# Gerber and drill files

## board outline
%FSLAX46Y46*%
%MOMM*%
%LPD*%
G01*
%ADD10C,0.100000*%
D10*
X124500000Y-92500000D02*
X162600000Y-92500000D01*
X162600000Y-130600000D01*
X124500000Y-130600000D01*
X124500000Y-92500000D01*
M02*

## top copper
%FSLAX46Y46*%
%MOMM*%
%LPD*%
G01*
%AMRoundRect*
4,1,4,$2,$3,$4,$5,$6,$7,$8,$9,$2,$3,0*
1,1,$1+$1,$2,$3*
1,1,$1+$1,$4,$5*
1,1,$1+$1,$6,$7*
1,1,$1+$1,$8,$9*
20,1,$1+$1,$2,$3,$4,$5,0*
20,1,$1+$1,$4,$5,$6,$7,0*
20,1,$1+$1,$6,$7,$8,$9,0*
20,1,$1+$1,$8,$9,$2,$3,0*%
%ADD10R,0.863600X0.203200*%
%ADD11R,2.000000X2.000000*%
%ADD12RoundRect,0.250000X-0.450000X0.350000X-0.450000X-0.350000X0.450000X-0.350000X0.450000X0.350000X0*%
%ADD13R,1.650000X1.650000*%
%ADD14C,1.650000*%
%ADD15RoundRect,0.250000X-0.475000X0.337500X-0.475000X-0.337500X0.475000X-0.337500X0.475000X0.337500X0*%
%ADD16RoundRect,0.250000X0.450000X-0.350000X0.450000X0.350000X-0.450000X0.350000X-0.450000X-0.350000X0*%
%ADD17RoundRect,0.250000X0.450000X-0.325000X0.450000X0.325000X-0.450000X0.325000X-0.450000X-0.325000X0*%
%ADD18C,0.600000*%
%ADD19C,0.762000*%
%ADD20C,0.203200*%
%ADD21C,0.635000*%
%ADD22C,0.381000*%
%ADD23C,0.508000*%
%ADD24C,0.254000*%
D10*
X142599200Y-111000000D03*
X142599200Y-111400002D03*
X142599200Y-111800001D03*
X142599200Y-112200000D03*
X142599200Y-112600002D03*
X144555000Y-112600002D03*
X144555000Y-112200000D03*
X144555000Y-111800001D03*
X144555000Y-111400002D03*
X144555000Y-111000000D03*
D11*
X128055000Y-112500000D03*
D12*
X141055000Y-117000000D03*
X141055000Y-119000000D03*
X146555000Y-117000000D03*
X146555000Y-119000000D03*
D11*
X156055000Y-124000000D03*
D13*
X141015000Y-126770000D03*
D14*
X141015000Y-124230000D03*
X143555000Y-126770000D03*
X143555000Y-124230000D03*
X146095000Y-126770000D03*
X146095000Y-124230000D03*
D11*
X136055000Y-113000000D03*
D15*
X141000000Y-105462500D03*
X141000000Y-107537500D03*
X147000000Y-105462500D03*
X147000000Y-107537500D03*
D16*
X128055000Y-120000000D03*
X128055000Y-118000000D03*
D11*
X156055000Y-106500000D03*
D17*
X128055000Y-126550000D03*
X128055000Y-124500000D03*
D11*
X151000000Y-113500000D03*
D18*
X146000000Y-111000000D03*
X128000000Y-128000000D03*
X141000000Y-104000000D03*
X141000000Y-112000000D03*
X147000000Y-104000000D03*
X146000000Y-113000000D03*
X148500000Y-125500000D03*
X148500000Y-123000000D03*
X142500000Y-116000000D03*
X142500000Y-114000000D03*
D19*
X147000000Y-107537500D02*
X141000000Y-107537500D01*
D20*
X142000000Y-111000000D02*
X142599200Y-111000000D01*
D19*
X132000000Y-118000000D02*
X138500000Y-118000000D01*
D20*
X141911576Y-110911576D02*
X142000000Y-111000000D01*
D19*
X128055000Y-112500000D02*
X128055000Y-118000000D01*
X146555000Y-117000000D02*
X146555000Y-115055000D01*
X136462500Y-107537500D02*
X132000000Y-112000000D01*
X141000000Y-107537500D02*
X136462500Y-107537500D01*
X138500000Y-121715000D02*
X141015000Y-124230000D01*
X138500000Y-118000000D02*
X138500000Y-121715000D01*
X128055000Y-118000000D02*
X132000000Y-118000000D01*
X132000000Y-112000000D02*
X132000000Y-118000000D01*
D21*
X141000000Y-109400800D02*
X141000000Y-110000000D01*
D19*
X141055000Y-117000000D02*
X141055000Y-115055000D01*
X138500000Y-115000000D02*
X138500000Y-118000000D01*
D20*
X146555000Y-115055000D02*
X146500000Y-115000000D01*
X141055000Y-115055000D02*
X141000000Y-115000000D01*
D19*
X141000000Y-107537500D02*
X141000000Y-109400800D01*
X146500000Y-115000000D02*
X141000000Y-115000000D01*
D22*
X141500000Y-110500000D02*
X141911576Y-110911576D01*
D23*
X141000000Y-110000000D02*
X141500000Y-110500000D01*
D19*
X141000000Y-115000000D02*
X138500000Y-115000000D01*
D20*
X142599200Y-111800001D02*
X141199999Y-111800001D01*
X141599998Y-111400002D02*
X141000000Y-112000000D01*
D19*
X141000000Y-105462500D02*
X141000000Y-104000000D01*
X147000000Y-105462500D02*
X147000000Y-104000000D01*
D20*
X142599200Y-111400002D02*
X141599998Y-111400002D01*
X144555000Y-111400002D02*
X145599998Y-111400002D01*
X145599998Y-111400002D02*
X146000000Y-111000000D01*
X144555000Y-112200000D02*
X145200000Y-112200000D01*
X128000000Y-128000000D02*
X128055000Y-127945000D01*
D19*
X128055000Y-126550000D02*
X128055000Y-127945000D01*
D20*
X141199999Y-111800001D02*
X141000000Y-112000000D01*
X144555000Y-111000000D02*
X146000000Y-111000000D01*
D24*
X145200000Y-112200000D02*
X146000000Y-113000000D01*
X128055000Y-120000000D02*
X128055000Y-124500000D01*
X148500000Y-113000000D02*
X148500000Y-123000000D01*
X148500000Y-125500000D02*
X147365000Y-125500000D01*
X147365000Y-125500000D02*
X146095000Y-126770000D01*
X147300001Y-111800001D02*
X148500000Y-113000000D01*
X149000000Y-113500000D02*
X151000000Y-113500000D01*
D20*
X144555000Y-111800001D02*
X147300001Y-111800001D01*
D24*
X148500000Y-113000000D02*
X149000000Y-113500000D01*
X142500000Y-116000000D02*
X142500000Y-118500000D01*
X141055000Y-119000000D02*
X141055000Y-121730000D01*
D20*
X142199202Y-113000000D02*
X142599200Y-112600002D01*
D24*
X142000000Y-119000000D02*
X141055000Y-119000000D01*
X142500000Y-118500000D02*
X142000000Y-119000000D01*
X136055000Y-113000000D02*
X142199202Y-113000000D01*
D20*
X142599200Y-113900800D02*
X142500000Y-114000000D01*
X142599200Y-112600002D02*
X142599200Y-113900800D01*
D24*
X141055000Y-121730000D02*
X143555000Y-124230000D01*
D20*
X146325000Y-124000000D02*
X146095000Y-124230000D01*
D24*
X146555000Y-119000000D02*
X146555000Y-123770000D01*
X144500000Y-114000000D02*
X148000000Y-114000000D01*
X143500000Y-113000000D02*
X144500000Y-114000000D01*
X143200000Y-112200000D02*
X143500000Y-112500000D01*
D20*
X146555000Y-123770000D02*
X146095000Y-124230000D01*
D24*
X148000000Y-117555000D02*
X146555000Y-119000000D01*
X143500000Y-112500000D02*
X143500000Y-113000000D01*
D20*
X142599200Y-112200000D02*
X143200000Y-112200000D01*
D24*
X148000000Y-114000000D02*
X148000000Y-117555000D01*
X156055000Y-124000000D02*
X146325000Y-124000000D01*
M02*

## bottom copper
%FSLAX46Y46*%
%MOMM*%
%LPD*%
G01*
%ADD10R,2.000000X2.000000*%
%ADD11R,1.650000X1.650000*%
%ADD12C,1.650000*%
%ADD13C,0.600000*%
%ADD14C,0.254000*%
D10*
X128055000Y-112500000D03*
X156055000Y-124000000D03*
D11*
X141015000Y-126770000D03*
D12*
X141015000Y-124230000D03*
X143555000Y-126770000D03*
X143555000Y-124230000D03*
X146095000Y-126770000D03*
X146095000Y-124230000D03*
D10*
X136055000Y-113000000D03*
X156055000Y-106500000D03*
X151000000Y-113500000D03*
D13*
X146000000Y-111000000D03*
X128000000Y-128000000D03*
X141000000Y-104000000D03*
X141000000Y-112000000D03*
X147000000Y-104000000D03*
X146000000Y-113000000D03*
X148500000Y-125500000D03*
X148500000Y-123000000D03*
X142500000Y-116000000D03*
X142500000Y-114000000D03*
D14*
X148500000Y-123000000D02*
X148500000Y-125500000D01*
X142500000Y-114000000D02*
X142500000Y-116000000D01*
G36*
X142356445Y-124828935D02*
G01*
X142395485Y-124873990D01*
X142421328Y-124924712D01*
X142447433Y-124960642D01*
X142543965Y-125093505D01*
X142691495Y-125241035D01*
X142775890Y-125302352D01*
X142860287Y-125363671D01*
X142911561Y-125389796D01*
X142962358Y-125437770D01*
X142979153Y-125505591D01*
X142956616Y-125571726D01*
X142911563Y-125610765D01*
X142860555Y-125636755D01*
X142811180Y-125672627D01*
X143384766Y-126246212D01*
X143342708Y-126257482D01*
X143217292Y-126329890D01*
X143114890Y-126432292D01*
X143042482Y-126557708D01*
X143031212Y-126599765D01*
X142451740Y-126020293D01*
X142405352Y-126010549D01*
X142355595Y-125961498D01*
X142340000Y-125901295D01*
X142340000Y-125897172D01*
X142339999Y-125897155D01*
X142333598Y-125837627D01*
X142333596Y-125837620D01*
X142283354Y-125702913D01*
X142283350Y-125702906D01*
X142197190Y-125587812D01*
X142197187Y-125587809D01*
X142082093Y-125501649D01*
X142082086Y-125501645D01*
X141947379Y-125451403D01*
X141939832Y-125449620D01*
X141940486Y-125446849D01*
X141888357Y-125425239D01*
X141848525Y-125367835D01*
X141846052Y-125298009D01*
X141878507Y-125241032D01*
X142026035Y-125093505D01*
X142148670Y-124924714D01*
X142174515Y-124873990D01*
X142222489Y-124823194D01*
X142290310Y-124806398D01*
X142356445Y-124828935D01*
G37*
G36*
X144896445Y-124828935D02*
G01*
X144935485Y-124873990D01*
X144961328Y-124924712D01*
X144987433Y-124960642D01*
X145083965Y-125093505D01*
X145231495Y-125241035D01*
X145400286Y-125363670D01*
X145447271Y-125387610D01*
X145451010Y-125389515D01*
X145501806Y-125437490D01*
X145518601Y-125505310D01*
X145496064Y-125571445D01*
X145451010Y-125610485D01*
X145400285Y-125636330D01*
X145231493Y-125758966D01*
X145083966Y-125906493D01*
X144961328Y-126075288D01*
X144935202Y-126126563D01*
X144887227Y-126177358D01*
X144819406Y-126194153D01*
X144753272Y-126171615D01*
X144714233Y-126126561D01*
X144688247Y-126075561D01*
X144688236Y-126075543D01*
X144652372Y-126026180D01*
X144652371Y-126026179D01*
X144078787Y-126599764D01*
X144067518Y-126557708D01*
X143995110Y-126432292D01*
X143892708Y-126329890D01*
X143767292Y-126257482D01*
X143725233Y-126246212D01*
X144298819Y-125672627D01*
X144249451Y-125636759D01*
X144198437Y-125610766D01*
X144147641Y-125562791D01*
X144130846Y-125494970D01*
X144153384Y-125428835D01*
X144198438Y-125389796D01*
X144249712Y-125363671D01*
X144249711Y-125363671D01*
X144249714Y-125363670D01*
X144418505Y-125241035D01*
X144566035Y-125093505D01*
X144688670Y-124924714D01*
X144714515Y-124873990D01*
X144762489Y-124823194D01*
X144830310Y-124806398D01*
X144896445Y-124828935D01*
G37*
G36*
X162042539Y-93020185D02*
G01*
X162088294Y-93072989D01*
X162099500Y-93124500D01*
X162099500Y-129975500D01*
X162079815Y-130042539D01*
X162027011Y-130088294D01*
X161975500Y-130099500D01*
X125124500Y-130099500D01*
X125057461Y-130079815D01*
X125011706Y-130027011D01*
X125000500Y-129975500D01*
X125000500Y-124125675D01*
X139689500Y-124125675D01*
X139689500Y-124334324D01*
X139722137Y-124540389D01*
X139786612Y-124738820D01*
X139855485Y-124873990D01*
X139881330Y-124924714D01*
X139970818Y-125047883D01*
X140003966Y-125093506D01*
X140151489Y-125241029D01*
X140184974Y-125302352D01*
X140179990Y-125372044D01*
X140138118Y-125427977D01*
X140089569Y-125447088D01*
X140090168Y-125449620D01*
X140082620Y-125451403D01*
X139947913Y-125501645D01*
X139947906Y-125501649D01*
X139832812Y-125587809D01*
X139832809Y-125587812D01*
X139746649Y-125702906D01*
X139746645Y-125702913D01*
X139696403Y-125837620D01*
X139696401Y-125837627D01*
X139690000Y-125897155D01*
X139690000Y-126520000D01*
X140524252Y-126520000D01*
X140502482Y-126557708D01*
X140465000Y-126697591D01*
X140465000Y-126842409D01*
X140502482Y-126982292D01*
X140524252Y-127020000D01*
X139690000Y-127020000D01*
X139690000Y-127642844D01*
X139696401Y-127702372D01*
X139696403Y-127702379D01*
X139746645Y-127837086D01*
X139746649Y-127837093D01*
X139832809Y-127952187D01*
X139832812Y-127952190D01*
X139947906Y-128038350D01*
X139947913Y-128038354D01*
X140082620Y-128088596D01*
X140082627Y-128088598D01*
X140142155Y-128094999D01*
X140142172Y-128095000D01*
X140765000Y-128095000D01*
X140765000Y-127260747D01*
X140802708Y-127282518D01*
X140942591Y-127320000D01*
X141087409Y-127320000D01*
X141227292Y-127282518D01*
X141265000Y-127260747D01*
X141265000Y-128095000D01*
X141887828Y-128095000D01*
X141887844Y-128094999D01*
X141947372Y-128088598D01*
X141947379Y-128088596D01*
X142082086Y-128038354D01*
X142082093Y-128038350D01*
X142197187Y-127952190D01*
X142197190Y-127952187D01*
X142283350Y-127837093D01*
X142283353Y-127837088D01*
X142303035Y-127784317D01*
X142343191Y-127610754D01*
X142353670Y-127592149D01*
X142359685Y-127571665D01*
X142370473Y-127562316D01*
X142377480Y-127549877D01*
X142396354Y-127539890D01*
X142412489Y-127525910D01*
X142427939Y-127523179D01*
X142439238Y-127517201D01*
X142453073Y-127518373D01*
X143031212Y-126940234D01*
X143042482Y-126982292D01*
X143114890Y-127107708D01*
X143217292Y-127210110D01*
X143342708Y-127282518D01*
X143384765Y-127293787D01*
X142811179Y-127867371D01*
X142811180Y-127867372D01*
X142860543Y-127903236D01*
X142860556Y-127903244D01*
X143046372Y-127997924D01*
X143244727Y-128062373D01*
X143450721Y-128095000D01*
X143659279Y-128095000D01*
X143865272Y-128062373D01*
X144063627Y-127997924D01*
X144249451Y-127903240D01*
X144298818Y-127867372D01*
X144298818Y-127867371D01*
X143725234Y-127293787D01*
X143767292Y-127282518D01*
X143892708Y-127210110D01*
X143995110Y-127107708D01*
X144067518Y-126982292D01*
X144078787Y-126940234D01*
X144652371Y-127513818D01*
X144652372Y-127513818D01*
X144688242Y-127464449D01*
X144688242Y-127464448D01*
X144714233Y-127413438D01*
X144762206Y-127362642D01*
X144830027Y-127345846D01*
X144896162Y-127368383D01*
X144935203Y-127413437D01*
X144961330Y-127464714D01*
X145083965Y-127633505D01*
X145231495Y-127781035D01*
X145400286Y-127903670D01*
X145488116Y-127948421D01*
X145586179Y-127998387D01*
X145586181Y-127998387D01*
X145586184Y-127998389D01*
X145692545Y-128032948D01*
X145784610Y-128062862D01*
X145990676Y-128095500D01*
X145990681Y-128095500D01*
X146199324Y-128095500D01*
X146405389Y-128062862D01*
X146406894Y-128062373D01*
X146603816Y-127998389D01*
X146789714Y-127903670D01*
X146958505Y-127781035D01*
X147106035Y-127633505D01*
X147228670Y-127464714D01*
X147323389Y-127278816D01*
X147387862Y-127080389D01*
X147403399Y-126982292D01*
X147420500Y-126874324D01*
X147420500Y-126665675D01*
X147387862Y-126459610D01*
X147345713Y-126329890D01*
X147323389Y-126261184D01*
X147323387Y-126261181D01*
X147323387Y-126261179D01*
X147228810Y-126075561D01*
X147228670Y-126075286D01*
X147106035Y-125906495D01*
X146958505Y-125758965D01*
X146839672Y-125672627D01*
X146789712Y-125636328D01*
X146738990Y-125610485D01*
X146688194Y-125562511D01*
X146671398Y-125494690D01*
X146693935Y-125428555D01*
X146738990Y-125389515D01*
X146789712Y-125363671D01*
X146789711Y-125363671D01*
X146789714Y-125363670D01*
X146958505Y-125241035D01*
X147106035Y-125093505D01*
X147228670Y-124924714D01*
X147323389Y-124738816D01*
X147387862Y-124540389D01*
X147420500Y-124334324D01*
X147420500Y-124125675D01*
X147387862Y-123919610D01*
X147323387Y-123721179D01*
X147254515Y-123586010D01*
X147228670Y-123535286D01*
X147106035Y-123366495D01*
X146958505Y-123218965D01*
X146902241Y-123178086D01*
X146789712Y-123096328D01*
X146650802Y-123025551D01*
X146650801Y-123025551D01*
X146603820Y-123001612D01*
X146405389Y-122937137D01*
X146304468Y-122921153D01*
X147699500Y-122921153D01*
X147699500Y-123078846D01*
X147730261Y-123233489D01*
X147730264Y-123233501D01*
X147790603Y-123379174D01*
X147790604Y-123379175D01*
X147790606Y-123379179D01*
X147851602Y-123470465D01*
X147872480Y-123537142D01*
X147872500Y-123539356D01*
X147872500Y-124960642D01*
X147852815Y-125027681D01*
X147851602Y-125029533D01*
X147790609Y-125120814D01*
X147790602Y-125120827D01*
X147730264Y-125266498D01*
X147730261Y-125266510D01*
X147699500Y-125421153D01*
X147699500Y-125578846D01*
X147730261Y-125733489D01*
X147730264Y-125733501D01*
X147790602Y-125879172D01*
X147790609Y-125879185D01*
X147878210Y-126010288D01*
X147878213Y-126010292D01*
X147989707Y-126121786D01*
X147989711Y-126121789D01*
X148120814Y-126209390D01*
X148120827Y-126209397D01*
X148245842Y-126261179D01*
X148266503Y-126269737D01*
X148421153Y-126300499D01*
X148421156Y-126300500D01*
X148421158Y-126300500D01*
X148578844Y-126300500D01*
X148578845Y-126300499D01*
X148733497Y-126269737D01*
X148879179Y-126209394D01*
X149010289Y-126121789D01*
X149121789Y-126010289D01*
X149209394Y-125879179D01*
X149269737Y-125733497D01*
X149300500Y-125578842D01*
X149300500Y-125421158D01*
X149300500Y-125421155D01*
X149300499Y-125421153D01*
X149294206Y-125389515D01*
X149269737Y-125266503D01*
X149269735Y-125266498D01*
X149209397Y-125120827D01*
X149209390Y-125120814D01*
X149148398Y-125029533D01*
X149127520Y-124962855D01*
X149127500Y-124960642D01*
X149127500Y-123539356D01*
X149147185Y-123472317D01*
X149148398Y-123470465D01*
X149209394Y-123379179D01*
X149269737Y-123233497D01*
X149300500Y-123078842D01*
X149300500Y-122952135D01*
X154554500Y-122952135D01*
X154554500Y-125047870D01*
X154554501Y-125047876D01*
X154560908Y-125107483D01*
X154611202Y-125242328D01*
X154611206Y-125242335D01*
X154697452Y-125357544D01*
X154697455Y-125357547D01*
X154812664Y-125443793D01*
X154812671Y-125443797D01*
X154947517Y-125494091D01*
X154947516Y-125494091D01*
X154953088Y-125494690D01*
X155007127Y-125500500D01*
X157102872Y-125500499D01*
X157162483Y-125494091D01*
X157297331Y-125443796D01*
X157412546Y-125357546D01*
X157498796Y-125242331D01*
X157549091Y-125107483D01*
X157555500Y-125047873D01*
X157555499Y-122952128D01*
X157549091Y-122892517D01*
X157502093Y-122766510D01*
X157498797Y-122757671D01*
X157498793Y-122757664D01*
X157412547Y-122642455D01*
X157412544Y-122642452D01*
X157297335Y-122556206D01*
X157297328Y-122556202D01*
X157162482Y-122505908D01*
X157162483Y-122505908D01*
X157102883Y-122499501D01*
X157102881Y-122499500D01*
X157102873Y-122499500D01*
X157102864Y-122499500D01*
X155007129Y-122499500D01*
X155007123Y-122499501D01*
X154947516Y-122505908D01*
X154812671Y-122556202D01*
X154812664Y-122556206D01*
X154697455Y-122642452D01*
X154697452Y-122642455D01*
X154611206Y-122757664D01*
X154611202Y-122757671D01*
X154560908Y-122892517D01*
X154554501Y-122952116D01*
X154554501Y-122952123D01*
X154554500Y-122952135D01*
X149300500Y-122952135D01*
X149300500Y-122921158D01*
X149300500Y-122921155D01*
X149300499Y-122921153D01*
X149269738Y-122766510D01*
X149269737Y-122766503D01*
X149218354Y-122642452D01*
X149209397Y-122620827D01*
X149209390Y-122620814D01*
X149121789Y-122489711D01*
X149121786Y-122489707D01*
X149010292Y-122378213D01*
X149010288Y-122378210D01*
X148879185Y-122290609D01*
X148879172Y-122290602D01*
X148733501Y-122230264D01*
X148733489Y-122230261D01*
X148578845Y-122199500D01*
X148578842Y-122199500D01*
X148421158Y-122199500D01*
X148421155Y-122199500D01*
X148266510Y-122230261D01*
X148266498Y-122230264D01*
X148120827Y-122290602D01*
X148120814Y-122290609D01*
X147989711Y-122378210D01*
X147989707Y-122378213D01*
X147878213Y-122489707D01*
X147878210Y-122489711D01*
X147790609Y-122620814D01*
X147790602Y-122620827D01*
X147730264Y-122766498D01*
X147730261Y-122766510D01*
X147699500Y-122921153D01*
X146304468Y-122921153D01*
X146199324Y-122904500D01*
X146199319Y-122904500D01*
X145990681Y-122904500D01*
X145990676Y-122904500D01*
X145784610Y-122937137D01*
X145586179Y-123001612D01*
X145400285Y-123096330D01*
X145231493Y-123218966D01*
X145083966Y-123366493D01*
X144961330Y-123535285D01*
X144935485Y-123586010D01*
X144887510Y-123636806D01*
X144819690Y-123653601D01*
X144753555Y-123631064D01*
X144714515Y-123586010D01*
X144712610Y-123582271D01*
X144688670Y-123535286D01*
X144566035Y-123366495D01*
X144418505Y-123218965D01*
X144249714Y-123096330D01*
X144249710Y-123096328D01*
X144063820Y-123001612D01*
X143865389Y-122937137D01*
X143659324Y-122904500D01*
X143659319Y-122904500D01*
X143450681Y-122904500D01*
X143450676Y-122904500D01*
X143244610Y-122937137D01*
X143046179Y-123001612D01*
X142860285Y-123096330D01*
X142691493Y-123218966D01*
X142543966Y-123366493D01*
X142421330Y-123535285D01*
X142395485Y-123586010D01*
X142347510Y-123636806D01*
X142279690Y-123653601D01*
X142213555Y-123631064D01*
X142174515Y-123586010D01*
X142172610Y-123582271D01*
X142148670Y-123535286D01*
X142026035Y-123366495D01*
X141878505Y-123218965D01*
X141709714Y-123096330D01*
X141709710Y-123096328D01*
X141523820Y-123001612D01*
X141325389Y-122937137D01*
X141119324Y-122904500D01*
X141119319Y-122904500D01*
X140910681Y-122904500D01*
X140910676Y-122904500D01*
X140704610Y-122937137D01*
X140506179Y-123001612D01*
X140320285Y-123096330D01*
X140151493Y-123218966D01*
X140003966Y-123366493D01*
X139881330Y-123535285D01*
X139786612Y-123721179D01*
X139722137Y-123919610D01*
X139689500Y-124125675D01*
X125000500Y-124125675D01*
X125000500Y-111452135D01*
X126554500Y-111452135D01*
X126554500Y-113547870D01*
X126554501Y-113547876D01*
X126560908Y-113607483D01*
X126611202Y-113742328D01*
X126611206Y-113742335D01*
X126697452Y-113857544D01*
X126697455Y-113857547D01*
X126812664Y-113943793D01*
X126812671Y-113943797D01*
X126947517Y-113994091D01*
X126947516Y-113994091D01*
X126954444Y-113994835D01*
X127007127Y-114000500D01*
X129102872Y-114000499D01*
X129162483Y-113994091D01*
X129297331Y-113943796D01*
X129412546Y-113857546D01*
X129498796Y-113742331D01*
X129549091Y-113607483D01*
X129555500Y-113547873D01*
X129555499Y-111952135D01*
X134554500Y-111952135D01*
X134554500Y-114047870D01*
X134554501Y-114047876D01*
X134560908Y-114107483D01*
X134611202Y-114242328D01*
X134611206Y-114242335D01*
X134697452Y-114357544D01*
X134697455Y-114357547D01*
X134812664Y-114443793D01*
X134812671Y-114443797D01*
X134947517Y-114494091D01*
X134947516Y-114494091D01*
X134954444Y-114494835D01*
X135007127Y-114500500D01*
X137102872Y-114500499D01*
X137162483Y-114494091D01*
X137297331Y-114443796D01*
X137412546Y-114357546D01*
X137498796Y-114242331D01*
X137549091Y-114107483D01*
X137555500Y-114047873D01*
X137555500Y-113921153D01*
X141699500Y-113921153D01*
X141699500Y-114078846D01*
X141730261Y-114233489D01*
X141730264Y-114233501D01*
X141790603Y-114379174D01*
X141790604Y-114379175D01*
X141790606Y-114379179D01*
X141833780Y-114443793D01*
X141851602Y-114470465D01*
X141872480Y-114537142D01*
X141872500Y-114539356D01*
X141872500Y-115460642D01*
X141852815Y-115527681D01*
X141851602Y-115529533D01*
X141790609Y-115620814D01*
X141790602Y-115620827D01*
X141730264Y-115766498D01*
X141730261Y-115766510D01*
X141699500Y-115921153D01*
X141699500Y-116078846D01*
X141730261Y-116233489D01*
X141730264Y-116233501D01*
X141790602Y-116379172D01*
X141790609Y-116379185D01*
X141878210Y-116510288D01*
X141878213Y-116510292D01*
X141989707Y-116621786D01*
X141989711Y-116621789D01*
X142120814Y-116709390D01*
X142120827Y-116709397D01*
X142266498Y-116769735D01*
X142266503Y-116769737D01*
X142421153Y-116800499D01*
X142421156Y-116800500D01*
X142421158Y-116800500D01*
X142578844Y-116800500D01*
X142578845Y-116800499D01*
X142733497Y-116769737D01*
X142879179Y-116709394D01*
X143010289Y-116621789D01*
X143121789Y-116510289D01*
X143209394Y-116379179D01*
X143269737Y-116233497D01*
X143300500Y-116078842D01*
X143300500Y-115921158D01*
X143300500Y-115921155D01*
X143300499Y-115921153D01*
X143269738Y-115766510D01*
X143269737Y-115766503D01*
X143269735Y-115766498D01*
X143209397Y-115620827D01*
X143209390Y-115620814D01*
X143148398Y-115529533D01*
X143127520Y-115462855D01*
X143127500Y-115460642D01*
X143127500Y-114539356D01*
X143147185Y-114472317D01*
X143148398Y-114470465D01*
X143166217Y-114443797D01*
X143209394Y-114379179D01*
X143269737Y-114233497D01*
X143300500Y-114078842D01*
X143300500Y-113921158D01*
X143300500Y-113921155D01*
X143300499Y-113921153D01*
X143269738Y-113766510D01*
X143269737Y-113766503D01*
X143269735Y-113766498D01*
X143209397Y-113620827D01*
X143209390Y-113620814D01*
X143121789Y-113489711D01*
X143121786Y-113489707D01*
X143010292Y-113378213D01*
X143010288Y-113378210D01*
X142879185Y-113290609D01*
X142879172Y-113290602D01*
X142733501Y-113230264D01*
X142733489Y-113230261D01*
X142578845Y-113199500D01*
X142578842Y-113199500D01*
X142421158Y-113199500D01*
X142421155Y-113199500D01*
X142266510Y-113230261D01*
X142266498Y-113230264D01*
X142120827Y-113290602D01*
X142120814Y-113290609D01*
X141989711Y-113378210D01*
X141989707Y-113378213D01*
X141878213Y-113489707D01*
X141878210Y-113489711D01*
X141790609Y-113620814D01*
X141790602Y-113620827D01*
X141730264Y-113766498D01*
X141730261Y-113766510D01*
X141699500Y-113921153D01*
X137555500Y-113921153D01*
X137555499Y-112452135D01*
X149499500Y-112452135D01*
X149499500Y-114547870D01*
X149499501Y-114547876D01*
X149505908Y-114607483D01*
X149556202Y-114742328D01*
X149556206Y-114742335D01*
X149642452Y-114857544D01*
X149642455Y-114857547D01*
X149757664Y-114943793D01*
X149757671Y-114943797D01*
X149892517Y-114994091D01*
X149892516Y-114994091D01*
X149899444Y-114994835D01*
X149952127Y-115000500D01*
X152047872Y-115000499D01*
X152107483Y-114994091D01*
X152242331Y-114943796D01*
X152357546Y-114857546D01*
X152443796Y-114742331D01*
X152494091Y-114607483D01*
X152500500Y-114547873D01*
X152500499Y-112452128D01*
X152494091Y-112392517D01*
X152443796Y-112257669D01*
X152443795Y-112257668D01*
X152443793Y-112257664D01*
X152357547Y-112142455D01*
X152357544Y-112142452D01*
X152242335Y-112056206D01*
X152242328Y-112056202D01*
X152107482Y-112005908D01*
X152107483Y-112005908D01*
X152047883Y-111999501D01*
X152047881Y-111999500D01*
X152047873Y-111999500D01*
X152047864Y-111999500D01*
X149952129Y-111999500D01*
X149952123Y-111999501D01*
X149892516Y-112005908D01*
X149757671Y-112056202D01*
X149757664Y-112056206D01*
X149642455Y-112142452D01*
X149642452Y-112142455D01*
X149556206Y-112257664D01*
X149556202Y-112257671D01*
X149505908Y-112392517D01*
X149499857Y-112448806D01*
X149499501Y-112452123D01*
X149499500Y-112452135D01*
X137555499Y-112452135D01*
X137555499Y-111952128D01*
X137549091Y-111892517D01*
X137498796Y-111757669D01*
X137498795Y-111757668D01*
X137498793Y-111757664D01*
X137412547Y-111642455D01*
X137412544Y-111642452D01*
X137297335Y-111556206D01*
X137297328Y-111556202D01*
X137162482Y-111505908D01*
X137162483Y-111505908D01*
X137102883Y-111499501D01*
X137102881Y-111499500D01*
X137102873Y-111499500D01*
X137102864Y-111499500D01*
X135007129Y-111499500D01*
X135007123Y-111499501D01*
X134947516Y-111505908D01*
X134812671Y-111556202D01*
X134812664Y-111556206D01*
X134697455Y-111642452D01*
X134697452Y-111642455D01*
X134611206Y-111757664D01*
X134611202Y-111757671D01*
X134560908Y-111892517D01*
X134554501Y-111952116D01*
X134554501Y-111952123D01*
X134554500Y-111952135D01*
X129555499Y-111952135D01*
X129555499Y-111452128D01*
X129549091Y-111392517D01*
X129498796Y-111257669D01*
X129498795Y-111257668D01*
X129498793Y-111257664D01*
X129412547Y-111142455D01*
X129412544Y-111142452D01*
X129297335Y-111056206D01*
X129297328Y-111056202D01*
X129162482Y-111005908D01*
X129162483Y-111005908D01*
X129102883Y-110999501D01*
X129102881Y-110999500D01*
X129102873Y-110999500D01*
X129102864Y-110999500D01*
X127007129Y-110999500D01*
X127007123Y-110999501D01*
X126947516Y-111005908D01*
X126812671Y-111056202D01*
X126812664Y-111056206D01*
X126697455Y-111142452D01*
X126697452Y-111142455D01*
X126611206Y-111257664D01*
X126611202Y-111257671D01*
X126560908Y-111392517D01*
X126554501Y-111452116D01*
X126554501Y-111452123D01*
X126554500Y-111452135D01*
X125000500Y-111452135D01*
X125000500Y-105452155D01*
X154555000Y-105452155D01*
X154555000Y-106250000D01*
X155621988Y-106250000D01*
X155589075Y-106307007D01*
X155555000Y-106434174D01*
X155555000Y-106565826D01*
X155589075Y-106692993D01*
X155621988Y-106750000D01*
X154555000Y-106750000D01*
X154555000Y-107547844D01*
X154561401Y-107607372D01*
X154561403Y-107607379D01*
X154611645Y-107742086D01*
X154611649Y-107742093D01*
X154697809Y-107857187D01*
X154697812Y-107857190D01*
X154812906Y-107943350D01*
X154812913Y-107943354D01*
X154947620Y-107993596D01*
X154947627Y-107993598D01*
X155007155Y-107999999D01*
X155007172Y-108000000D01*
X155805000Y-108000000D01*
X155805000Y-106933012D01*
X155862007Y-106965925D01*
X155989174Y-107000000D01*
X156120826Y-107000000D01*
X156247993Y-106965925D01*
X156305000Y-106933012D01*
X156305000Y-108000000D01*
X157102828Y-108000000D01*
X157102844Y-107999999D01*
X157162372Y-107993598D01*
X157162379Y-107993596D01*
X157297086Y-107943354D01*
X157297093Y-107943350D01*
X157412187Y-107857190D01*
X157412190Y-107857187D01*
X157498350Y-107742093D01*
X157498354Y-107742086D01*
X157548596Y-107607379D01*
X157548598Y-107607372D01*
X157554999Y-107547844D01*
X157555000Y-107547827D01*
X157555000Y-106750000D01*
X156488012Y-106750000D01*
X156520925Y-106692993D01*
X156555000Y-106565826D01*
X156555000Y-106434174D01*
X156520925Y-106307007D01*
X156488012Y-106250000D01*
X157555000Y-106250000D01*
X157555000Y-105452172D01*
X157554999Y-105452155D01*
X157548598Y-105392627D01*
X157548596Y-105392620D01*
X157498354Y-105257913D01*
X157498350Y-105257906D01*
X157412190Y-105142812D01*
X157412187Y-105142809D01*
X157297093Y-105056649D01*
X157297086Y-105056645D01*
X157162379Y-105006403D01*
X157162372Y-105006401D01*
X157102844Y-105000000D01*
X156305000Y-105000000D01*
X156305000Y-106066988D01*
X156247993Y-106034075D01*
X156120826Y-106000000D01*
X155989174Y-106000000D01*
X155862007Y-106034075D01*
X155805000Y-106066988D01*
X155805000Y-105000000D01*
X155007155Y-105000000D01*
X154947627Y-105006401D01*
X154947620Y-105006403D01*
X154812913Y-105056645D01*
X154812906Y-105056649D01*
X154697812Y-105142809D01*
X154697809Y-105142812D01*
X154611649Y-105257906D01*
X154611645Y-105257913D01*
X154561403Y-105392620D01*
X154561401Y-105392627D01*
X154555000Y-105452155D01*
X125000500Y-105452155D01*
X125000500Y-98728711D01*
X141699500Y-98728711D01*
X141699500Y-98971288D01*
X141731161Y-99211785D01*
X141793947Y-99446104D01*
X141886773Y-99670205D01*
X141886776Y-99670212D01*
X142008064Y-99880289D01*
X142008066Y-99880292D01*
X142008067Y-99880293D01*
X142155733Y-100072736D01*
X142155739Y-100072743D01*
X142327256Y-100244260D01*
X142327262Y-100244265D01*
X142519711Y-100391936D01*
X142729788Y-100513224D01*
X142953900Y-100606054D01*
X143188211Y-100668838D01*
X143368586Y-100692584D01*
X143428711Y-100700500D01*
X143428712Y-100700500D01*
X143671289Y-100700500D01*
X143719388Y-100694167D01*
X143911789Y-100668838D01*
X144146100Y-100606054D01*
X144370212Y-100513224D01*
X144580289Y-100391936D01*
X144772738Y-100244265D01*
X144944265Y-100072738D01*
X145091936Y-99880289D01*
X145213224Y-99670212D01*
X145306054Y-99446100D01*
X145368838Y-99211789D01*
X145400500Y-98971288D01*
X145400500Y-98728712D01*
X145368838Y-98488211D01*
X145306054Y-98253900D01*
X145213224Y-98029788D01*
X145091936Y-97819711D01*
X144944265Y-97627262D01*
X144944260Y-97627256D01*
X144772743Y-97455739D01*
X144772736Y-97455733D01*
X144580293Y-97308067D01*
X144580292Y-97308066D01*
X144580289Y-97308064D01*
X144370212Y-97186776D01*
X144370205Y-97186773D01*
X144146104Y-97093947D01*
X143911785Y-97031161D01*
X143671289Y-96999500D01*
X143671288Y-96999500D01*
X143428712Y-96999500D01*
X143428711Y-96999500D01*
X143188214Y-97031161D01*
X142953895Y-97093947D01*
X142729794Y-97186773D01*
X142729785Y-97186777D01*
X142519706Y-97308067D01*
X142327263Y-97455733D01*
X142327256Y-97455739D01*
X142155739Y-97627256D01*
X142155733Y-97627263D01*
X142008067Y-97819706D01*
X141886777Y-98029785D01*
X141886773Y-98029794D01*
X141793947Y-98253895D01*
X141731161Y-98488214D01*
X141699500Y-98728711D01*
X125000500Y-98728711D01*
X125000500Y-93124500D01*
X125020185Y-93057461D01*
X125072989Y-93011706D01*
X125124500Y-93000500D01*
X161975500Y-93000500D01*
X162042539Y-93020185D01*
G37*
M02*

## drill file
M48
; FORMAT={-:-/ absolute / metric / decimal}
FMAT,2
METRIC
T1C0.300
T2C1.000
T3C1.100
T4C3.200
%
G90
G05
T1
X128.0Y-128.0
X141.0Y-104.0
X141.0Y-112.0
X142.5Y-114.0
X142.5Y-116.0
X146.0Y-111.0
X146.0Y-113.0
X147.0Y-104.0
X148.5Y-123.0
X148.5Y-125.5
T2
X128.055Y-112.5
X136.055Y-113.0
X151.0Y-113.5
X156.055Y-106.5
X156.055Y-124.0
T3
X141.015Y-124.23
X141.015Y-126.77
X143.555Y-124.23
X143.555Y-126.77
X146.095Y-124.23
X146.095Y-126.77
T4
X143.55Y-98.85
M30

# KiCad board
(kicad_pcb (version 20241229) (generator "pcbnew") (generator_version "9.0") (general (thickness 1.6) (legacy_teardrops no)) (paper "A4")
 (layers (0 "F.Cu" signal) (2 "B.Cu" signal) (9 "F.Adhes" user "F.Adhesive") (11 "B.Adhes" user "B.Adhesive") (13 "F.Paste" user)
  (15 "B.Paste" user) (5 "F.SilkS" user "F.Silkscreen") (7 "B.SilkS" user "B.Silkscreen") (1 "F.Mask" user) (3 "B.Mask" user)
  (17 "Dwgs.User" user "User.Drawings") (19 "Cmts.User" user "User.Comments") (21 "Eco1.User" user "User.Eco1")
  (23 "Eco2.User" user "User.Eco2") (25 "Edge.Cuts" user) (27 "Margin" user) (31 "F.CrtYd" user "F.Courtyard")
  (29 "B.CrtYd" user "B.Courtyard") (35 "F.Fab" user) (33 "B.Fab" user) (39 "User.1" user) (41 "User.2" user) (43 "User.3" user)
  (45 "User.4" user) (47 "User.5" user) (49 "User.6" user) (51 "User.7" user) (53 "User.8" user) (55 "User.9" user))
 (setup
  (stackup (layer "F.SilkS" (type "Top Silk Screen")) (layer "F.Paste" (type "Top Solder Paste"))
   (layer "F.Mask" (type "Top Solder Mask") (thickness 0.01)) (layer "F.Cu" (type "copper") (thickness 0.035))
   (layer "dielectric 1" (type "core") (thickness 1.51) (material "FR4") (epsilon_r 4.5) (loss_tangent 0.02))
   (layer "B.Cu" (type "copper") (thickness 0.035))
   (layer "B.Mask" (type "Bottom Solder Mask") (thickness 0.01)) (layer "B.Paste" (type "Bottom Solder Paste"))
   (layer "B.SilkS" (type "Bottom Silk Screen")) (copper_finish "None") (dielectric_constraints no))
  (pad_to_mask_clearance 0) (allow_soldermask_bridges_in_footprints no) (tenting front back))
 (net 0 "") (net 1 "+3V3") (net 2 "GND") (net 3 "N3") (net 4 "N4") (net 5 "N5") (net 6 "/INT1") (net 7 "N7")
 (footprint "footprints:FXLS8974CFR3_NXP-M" (layer "F.Cu") (at 143.5771 111.800001)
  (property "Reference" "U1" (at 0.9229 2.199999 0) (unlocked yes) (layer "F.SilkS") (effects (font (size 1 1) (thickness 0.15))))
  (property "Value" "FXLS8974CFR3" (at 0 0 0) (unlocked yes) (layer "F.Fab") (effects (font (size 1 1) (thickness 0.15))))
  (pad "1" smd rect (at -0.9779 -0.800001) (size 0.8636 0.2032) (layers "F.Cu" "F.Mask" "F.Paste") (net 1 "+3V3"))
  (pad "2" smd rect (at -0.9779 -0.399999) (size 0.8636 0.2032) (layers "F.Cu" "F.Mask" "F.Paste") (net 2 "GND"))
  (pad "3" smd rect (at -0.9779 0) (size 0.8636 0.2032) (layers "F.Cu" "F.Mask" "F.Paste") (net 2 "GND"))
  (pad "4" smd rect (at -0.9779 0.399999) (size 0.8636 0.2032) (layers "F.Cu" "F.Mask" "F.Paste") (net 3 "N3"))
  (pad "5" smd rect (at -0.9779 0.800001) (size 0.8636 0.2032) (layers "F.Cu" "F.Mask" "F.Paste") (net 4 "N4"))
  (pad "6" smd rect (at 0.9779 0.800001) (size 0.8636 0.2032) (layers "F.Cu" "F.Mask" "F.Paste") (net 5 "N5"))
  (pad "7" smd rect (at 0.9779 0.399999) (size 0.8636 0.2032) (layers "F.Cu" "F.Mask" "F.Paste") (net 2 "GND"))
  (pad "8" smd rect (at 0.9779 0) (size 0.8636 0.2032) (layers "F.Cu" "F.Mask" "F.Paste") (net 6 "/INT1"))
  (pad "9" smd rect (at 0.9779 -0.399999) (size 0.8636 0.2032) (layers "F.Cu" "F.Mask" "F.Paste") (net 2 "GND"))
  (pad "10" smd rect (at 0.9779 -0.800001) (size 0.8636 0.2032) (layers "F.Cu" "F.Mask" "F.Paste") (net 2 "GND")))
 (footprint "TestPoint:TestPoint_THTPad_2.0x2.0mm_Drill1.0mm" (layer "F.Cu") (at 128.055 112.5)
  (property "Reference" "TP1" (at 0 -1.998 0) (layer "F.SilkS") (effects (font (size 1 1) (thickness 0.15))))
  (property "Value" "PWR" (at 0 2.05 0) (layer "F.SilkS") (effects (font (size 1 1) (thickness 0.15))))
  (pad "1" thru_hole rect (at 0 0) (size 2 2) (drill 1) (layers "*.Cu" "*.Mask") (remove_unused_layers no) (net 1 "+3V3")))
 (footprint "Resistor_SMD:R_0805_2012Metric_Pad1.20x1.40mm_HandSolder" (layer "F.Cu") (at 141.055 118 -90)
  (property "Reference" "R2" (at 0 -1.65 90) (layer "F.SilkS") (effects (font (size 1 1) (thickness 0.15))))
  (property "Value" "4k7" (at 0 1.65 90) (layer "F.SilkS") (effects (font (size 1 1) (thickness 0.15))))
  (pad "1" smd roundrect (at -1 0 270) (size 1.2 1.4) (layers "F.Cu" "F.Mask" "F.Paste") (roundrect_rratio 0.208333) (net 1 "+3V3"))
  (pad "2" smd roundrect (at 1 0 270) (size 1.2 1.4) (layers "F.Cu" "F.Mask" "F.Paste") (roundrect_rratio 0.208333) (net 4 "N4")))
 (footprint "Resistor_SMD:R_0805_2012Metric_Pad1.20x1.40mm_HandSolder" (layer "F.Cu") (at 146.555 118 -90)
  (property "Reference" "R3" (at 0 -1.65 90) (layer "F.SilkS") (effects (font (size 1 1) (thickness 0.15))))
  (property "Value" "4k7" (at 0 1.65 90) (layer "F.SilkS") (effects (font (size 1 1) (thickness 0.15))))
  (pad "1" smd roundrect (at -1 0 270) (size 1.2 1.4) (layers "F.Cu" "F.Mask" "F.Paste") (roundrect_rratio 0.208333) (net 1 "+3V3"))
  (pad "2" smd roundrect (at 1 0 270) (size 1.2 1.4) (layers "F.Cu" "F.Mask" "F.Paste") (roundrect_rratio 0.208333) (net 3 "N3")))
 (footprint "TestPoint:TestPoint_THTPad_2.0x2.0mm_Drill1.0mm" (layer "F.Cu") (at 156.055 124)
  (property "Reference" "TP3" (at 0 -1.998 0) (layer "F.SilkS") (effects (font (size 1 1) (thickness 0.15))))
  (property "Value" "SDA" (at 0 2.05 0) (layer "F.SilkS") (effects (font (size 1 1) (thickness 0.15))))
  (pad "1" thru_hole rect (at 0 0) (size 2 2) (drill 1) (layers "*.Cu" "*.Mask") (remove_unused_layers no) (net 3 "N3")))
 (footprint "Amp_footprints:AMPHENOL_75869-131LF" (layer "F.Cu") (at 143.555 125.5)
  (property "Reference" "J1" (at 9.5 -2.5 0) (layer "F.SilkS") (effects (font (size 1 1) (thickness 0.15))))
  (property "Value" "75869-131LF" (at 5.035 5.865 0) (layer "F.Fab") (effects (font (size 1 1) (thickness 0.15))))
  (pad "01" thru_hole rect (at -2.54 1.27) (size 1.65 1.65) (drill 1.1) (layers "*.Cu" "*.Mask") (remove_unused_layers no) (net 2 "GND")
   (solder_mask_margin 0.102))
  (pad "02" thru_hole circle (at -2.54 -1.27) (size 1.65 1.65) (drill 1.1) (layers "*.Cu" "*.Mask") (remove_unused_layers no) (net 1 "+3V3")
   (solder_mask_margin 0.102))
  (pad "03" thru_hole circle (at 0 1.27) (size 1.65 1.65) (drill 1.1) (layers "*.Cu" "*.Mask") (remove_unused_layers no) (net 2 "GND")
   (solder_mask_margin 0.102))
  (pad "04" thru_hole circle (at 0 -1.27) (size 1.65 1.65) (drill 1.1) (layers "*.Cu" "*.Mask") (remove_unused_layers no) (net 4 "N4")
   (solder_mask_margin 0.102))
  (pad "05" thru_hole circle (at 2.54 1.27) (size 1.65 1.65) (drill 1.1) (layers "*.Cu" "*.Mask") (remove_unused_layers no) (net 6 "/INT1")
   (solder_mask_margin 0.102))
  (pad "06" thru_hole circle (at 2.54 -1.27) (size 1.65 1.65) (drill 1.1) (layers "*.Cu" "*.Mask") (remove_unused_layers no) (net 3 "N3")
   (solder_mask_margin 0.102)))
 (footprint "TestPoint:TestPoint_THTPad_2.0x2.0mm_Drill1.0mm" (layer "F.Cu") (at 136.055 113 90)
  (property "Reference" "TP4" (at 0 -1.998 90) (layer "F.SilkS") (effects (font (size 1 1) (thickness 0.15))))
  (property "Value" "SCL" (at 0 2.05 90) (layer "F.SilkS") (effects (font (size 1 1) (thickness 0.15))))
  (pad "1" thru_hole rect (at 0 0 90) (size 2 2) (drill 1) (layers "*.Cu" "*.Mask") (remove_unused_layers no) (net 4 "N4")))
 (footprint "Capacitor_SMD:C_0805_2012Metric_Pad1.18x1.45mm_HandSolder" (layer "F.Cu") (at 141 106.5 -90)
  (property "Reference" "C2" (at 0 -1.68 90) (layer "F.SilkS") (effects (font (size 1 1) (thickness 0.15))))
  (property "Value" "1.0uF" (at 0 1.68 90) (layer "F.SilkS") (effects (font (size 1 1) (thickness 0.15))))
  (pad "1" smd roundrect (at -1.0375 0 270) (size 1.175 1.45) (layers "F.Cu" "F.Mask" "F.Paste") (roundrect_rratio 0.212766) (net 2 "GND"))
  (pad "2" smd roundrect (at 1.0375 0 270) (size 1.175 1.45) (layers "F.Cu" "F.Mask" "F.Paste") (roundrect_rratio 0.212766) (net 1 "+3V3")))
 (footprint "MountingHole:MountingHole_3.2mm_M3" (layer "F.Cu") (at 143.55 98.85)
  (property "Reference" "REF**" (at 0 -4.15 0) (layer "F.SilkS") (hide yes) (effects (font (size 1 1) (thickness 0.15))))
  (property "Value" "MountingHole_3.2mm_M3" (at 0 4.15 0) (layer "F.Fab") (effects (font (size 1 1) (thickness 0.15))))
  (pad "" np_thru_hole circle (at 0 0) (size 3.2 3.2) (drill 3.2) (layers "*.Cu" "*.Mask")))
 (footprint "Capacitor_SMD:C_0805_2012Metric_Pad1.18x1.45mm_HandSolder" (layer "F.Cu") (at 147 106.5 -90)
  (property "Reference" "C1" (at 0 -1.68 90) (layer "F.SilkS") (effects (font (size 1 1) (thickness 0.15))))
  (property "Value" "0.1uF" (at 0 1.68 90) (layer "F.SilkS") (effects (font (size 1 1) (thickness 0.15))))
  (pad "1" smd roundrect (at -1.0375 0 270) (size 1.175 1.45) (layers "F.Cu" "F.Mask" "F.Paste") (roundrect_rratio 0.212766) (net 2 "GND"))
  (pad "2" smd roundrect (at 1.0375 0 270) (size 1.175 1.45) (layers "F.Cu" "F.Mask" "F.Paste") (roundrect_rratio 0.212766) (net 1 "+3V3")))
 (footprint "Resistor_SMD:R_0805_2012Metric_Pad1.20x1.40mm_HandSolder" (layer "F.Cu") (at 128.055 119 90)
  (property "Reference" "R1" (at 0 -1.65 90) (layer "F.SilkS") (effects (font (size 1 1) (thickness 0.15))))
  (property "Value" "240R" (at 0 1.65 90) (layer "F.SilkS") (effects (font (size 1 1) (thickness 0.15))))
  (pad "1" smd roundrect (at -1 0 90) (size 1.2 1.4) (layers "F.Cu" "F.Mask" "F.Paste") (roundrect_rratio 0.208333) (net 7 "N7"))
  (pad "2" smd roundrect (at 1 0 90) (size 1.2 1.4) (layers "F.Cu" "F.Mask" "F.Paste") (roundrect_rratio 0.208333) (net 1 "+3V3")))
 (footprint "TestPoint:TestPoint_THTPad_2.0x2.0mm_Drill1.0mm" (layer "F.Cu") (at 156.055 106.5)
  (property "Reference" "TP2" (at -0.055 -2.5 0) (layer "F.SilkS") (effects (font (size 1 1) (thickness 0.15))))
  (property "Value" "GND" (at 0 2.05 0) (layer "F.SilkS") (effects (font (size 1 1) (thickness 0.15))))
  (pad "1" thru_hole rect (at 0 0) (size 2 2) (drill 1) (layers "*.Cu" "*.Mask") (remove_unused_layers no) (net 2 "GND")))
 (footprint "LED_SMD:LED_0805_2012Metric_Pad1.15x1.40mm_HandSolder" (layer "F.Cu") (at 128.055 125.525 90)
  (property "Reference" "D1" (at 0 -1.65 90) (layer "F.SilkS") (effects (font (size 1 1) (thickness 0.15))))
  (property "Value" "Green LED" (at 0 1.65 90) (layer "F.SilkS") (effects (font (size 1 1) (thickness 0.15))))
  (pad "1" smd roundrect (at -1.025 0 90) (size 1.15 1.4) (layers "F.Cu" "F.Mask" "F.Paste") (roundrect_rratio 0.217391) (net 2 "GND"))
  (pad "2" smd roundrect (at 1.025 0 90) (size 1.15 1.4) (layers "F.Cu" "F.Mask" "F.Paste") (roundrect_rratio 0.217391) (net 7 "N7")))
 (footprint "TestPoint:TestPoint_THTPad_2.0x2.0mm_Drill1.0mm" (layer "F.Cu") (at 151 113.5)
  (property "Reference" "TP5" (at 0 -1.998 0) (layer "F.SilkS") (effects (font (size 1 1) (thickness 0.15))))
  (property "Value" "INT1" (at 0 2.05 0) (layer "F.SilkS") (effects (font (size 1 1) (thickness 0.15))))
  (pad "1" thru_hole rect (at 0 0) (size 2 2) (drill 1) (layers "*.Cu" "*.Mask") (remove_unused_layers no) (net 6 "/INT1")))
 (gr_rect (start 124.5 92.5) (end 162.6 130.6) (stroke (width 0.1) (type solid)) (fill no) (layer "Edge.Cuts"))
 (segment (start 147 107.5375) (end 141 107.5375) (width 0.762) (layer "F.Cu") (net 1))
 (segment (start 142 111) (end 142.5992 111) (width 0.2032) (layer "F.Cu") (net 1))
 (segment (start 132 118) (end 138.5 118) (width 0.762) (layer "F.Cu") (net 1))
 (segment (start 141.911576 110.911576) (end 142 111) (width 0.2032) (layer "F.Cu") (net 1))
 (segment (start 128.055 112.5) (end 128.055 118) (width 0.762) (layer "F.Cu") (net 1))
 (segment (start 146.555 117) (end 146.555 115.055) (width 0.762) (layer "F.Cu") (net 1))
 (segment (start 136.4625 107.5375) (end 132 112) (width 0.762) (layer "F.Cu") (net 1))
 (segment (start 141 107.5375) (end 136.4625 107.5375) (width 0.762) (layer "F.Cu") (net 1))
 (segment (start 138.5 121.715) (end 141.015 124.23) (width 0.762) (layer "F.Cu") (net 1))
 (segment (start 138.5 118) (end 138.5 121.715) (width 0.762) (layer "F.Cu") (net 1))
 (segment (start 128.055 118) (end 132 118) (width 0.762) (layer "F.Cu") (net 1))
 (segment (start 132 112) (end 132 118) (width 0.762) (layer "F.Cu") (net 1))
 (segment (start 141 109.4008) (end 141 110) (width 0.635) (layer "F.Cu") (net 1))
 (segment (start 141.055 117) (end 141.055 115.055) (width 0.762) (layer "F.Cu") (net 1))
 (segment (start 138.5 115) (end 138.5 118) (width 0.762) (layer "F.Cu") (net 1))
 (segment (start 146.555 115.055) (end 146.5 115) (width 0.2032) (layer "F.Cu") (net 1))
 (segment (start 141.055 115.055) (end 141 115) (width 0.2032) (layer "F.Cu") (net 1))
 (segment (start 141 107.5375) (end 141 109.4008) (width 0.762) (layer "F.Cu") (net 1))
 (segment (start 146.5 115) (end 141 115) (width 0.762) (layer "F.Cu") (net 1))
 (segment (start 141.5 110.5) (end 141.911576 110.911576) (width 0.381) (layer "F.Cu") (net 1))
 (segment (start 141 110) (end 141.5 110.5) (width 0.508) (layer "F.Cu") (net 1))
 (segment (start 141 115) (end 138.5 115) (width 0.762) (layer "F.Cu") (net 1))
 (segment (start 142.5992 111.800001) (end 141.199999 111.800001) (width 0.2032) (layer "F.Cu") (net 2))
 (segment (start 141.599998 111.400002) (end 141 112) (width 0.2032) (layer "F.Cu") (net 2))
 (segment (start 141 105.4625) (end 141 104) (width 0.762) (layer "F.Cu") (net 2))
 (segment (start 147 105.4625) (end 147 104) (width 0.762) (layer "F.Cu") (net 2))
 (segment (start 142.5992 111.400002) (end 141.599998 111.400002) (width 0.2032) (layer "F.Cu") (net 2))
 (segment (start 144.555 111.400002) (end 145.599998 111.400002) (width 0.2032) (layer "F.Cu") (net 2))
 (segment (start 145.599998 111.400002) (end 146 111) (width 0.2032) (layer "F.Cu") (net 2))
 (segment (start 144.555 112.2) (end 145.2 112.2) (width 0.2032) (layer "F.Cu") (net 2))
 (segment (start 128 128) (end 128.055 127.945) (width 0.2032) (layer "F.Cu") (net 2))
 (segment (start 128.055 126.55) (end 128.055 127.945) (width 0.762) (layer "F.Cu") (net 2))
 (segment (start 141.199999 111.800001) (end 141 112) (width 0.2032) (layer "F.Cu") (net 2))
 (segment (start 144.555 111) (end 146 111) (width 0.2032) (layer "F.Cu") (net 2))
 (segment (start 145.2 112.2) (end 146 113) (width 0.254) (layer "F.Cu") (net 2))
 (via (at 146 111) (size 0.6) (drill 0.3) (layers "F.Cu" "B.Cu") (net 2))
 (via (at 128 128) (size 0.6) (drill 0.3) (layers "F.Cu" "B.Cu") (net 2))
 (via (at 141 104) (size 0.6) (drill 0.3) (layers "F.Cu" "B.Cu") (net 2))
 (via (at 141 112) (size 0.6) (drill 0.3) (layers "F.Cu" "B.Cu") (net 2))
 (via (at 147 104) (size 0.6) (drill 0.3) (layers "F.Cu" "B.Cu") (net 2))
 (via (at 146 113) (size 0.6) (drill 0.3) (layers "F.Cu" "B.Cu") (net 2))
 (segment (start 128.055 120) (end 128.055 124.5) (width 0.254) (layer "F.Cu") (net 7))
 (segment (start 148.5 113) (end 148.5 123) (width 0.254) (layer "F.Cu") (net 6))
 (segment (start 148.5 125.5) (end 147.365 125.5) (width 0.254) (layer "F.Cu") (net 6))
 (segment (start 147.365 125.5) (end 146.095 126.77) (width 0.254) (layer "F.Cu") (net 6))
 (segment (start 147.300001 111.800001) (end 148.5 113) (width 0.254) (layer "F.Cu") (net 6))
 (segment (start 149 113.5) (end 151 113.5) (width 0.254) (layer "F.Cu") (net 6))
 (segment (start 144.555 111.800001) (end 147.300001 111.800001) (width 0.2032) (layer "F.Cu") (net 6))
 (segment (start 148.5 113) (end 149 113.5) (width 0.254) (layer "F.Cu") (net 6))
 (via (at 148.5 125.5) (size 0.6) (drill 0.3) (layers "F.Cu" "B.Cu") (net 6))
 (via (at 148.5 123) (size 0.6) (drill 0.3) (layers "F.Cu" "B.Cu") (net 6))
 (segment (start 148.5 123) (end 148.5 125.5) (width 0.254) (layer "B.Cu") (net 6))
 (segment (start 142.5 116) (end 142.5 118.5) (width 0.254) (layer "F.Cu") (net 4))
 (segment (start 141.055 119) (end 141.055 121.73) (width 0.254) (layer "F.Cu") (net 4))
 (segment (start 142.199202 113) (end 142.5992 112.600002) (width 0.2032) (layer "F.Cu") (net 4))
 (segment (start 142 119) (end 141.055 119) (width 0.254) (layer "F.Cu") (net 4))
 (segment (start 142.5 118.5) (end 142 119) (width 0.254) (layer "F.Cu") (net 4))
 (segment (start 136.055 113) (end 142.199202 113) (width 0.254) (layer "F.Cu") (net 4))
 (segment (start 142.5992 113.9008) (end 142.5 114) (width 0.2032) (layer "F.Cu") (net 4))
 (segment (start 142.5992 112.600002) (end 142.5992 113.9008) (width 0.2032) (layer "F.Cu") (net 4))
 (segment (start 141.055 121.73) (end 143.555 124.23) (width 0.254) (layer "F.Cu") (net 4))
 (via (at 142.5 116) (size 0.6) (drill 0.3) (layers "F.Cu" "B.Cu") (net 4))
 (via (at 142.5 114) (size 0.6) (drill 0.3) (layers "F.Cu" "B.Cu") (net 4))
 (segment (start 142.5 114) (end 142.5 116) (width 0.254) (layer "B.Cu") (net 4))
 (segment (start 146.325 124) (end 146.095 124.23) (width 0.2032) (layer "F.Cu") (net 3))
 (segment (start 146.555 119) (end 146.555 123.77) (width 0.254) (layer "F.Cu") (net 3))
 (segment (start 144.5 114) (end 148 114) (width 0.254) (layer "F.Cu") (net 3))
 (segment (start 143.5 113) (end 144.5 114) (width 0.254) (layer "F.Cu") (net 3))
 (segment (start 143.2 112.2) (end 143.5 112.5) (width 0.254) (layer "F.Cu") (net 3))
 (segment (start 146.555 123.77) (end 146.095 124.23) (width 0.2032) (layer "F.Cu") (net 3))
 (segment (start 148 117.555) (end 146.555 119) (width 0.254) (layer "F.Cu") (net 3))
 (segment (start 143.5 112.5) (end 143.5 113) (width 0.254) (layer "F.Cu") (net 3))
 (segment (start 142.5992 112.2) (end 143.2 112.2) (width 0.2032) (layer "F.Cu") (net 3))
 (segment (start 148 114) (end 148 117.555) (width 0.254) (layer "F.Cu") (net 3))
 (segment (start 156.055 124) (end 146.325 124) (width 0.254) (layer "F.Cu") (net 3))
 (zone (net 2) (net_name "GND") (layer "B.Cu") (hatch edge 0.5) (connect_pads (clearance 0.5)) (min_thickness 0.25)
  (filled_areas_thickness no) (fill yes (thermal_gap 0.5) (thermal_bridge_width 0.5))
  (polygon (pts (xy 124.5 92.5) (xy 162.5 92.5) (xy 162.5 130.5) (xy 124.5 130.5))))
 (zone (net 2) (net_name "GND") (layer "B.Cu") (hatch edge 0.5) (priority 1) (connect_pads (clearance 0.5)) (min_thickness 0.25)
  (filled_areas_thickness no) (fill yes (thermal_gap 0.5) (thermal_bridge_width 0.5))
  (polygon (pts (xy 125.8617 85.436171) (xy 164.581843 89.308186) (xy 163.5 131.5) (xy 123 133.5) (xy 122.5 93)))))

